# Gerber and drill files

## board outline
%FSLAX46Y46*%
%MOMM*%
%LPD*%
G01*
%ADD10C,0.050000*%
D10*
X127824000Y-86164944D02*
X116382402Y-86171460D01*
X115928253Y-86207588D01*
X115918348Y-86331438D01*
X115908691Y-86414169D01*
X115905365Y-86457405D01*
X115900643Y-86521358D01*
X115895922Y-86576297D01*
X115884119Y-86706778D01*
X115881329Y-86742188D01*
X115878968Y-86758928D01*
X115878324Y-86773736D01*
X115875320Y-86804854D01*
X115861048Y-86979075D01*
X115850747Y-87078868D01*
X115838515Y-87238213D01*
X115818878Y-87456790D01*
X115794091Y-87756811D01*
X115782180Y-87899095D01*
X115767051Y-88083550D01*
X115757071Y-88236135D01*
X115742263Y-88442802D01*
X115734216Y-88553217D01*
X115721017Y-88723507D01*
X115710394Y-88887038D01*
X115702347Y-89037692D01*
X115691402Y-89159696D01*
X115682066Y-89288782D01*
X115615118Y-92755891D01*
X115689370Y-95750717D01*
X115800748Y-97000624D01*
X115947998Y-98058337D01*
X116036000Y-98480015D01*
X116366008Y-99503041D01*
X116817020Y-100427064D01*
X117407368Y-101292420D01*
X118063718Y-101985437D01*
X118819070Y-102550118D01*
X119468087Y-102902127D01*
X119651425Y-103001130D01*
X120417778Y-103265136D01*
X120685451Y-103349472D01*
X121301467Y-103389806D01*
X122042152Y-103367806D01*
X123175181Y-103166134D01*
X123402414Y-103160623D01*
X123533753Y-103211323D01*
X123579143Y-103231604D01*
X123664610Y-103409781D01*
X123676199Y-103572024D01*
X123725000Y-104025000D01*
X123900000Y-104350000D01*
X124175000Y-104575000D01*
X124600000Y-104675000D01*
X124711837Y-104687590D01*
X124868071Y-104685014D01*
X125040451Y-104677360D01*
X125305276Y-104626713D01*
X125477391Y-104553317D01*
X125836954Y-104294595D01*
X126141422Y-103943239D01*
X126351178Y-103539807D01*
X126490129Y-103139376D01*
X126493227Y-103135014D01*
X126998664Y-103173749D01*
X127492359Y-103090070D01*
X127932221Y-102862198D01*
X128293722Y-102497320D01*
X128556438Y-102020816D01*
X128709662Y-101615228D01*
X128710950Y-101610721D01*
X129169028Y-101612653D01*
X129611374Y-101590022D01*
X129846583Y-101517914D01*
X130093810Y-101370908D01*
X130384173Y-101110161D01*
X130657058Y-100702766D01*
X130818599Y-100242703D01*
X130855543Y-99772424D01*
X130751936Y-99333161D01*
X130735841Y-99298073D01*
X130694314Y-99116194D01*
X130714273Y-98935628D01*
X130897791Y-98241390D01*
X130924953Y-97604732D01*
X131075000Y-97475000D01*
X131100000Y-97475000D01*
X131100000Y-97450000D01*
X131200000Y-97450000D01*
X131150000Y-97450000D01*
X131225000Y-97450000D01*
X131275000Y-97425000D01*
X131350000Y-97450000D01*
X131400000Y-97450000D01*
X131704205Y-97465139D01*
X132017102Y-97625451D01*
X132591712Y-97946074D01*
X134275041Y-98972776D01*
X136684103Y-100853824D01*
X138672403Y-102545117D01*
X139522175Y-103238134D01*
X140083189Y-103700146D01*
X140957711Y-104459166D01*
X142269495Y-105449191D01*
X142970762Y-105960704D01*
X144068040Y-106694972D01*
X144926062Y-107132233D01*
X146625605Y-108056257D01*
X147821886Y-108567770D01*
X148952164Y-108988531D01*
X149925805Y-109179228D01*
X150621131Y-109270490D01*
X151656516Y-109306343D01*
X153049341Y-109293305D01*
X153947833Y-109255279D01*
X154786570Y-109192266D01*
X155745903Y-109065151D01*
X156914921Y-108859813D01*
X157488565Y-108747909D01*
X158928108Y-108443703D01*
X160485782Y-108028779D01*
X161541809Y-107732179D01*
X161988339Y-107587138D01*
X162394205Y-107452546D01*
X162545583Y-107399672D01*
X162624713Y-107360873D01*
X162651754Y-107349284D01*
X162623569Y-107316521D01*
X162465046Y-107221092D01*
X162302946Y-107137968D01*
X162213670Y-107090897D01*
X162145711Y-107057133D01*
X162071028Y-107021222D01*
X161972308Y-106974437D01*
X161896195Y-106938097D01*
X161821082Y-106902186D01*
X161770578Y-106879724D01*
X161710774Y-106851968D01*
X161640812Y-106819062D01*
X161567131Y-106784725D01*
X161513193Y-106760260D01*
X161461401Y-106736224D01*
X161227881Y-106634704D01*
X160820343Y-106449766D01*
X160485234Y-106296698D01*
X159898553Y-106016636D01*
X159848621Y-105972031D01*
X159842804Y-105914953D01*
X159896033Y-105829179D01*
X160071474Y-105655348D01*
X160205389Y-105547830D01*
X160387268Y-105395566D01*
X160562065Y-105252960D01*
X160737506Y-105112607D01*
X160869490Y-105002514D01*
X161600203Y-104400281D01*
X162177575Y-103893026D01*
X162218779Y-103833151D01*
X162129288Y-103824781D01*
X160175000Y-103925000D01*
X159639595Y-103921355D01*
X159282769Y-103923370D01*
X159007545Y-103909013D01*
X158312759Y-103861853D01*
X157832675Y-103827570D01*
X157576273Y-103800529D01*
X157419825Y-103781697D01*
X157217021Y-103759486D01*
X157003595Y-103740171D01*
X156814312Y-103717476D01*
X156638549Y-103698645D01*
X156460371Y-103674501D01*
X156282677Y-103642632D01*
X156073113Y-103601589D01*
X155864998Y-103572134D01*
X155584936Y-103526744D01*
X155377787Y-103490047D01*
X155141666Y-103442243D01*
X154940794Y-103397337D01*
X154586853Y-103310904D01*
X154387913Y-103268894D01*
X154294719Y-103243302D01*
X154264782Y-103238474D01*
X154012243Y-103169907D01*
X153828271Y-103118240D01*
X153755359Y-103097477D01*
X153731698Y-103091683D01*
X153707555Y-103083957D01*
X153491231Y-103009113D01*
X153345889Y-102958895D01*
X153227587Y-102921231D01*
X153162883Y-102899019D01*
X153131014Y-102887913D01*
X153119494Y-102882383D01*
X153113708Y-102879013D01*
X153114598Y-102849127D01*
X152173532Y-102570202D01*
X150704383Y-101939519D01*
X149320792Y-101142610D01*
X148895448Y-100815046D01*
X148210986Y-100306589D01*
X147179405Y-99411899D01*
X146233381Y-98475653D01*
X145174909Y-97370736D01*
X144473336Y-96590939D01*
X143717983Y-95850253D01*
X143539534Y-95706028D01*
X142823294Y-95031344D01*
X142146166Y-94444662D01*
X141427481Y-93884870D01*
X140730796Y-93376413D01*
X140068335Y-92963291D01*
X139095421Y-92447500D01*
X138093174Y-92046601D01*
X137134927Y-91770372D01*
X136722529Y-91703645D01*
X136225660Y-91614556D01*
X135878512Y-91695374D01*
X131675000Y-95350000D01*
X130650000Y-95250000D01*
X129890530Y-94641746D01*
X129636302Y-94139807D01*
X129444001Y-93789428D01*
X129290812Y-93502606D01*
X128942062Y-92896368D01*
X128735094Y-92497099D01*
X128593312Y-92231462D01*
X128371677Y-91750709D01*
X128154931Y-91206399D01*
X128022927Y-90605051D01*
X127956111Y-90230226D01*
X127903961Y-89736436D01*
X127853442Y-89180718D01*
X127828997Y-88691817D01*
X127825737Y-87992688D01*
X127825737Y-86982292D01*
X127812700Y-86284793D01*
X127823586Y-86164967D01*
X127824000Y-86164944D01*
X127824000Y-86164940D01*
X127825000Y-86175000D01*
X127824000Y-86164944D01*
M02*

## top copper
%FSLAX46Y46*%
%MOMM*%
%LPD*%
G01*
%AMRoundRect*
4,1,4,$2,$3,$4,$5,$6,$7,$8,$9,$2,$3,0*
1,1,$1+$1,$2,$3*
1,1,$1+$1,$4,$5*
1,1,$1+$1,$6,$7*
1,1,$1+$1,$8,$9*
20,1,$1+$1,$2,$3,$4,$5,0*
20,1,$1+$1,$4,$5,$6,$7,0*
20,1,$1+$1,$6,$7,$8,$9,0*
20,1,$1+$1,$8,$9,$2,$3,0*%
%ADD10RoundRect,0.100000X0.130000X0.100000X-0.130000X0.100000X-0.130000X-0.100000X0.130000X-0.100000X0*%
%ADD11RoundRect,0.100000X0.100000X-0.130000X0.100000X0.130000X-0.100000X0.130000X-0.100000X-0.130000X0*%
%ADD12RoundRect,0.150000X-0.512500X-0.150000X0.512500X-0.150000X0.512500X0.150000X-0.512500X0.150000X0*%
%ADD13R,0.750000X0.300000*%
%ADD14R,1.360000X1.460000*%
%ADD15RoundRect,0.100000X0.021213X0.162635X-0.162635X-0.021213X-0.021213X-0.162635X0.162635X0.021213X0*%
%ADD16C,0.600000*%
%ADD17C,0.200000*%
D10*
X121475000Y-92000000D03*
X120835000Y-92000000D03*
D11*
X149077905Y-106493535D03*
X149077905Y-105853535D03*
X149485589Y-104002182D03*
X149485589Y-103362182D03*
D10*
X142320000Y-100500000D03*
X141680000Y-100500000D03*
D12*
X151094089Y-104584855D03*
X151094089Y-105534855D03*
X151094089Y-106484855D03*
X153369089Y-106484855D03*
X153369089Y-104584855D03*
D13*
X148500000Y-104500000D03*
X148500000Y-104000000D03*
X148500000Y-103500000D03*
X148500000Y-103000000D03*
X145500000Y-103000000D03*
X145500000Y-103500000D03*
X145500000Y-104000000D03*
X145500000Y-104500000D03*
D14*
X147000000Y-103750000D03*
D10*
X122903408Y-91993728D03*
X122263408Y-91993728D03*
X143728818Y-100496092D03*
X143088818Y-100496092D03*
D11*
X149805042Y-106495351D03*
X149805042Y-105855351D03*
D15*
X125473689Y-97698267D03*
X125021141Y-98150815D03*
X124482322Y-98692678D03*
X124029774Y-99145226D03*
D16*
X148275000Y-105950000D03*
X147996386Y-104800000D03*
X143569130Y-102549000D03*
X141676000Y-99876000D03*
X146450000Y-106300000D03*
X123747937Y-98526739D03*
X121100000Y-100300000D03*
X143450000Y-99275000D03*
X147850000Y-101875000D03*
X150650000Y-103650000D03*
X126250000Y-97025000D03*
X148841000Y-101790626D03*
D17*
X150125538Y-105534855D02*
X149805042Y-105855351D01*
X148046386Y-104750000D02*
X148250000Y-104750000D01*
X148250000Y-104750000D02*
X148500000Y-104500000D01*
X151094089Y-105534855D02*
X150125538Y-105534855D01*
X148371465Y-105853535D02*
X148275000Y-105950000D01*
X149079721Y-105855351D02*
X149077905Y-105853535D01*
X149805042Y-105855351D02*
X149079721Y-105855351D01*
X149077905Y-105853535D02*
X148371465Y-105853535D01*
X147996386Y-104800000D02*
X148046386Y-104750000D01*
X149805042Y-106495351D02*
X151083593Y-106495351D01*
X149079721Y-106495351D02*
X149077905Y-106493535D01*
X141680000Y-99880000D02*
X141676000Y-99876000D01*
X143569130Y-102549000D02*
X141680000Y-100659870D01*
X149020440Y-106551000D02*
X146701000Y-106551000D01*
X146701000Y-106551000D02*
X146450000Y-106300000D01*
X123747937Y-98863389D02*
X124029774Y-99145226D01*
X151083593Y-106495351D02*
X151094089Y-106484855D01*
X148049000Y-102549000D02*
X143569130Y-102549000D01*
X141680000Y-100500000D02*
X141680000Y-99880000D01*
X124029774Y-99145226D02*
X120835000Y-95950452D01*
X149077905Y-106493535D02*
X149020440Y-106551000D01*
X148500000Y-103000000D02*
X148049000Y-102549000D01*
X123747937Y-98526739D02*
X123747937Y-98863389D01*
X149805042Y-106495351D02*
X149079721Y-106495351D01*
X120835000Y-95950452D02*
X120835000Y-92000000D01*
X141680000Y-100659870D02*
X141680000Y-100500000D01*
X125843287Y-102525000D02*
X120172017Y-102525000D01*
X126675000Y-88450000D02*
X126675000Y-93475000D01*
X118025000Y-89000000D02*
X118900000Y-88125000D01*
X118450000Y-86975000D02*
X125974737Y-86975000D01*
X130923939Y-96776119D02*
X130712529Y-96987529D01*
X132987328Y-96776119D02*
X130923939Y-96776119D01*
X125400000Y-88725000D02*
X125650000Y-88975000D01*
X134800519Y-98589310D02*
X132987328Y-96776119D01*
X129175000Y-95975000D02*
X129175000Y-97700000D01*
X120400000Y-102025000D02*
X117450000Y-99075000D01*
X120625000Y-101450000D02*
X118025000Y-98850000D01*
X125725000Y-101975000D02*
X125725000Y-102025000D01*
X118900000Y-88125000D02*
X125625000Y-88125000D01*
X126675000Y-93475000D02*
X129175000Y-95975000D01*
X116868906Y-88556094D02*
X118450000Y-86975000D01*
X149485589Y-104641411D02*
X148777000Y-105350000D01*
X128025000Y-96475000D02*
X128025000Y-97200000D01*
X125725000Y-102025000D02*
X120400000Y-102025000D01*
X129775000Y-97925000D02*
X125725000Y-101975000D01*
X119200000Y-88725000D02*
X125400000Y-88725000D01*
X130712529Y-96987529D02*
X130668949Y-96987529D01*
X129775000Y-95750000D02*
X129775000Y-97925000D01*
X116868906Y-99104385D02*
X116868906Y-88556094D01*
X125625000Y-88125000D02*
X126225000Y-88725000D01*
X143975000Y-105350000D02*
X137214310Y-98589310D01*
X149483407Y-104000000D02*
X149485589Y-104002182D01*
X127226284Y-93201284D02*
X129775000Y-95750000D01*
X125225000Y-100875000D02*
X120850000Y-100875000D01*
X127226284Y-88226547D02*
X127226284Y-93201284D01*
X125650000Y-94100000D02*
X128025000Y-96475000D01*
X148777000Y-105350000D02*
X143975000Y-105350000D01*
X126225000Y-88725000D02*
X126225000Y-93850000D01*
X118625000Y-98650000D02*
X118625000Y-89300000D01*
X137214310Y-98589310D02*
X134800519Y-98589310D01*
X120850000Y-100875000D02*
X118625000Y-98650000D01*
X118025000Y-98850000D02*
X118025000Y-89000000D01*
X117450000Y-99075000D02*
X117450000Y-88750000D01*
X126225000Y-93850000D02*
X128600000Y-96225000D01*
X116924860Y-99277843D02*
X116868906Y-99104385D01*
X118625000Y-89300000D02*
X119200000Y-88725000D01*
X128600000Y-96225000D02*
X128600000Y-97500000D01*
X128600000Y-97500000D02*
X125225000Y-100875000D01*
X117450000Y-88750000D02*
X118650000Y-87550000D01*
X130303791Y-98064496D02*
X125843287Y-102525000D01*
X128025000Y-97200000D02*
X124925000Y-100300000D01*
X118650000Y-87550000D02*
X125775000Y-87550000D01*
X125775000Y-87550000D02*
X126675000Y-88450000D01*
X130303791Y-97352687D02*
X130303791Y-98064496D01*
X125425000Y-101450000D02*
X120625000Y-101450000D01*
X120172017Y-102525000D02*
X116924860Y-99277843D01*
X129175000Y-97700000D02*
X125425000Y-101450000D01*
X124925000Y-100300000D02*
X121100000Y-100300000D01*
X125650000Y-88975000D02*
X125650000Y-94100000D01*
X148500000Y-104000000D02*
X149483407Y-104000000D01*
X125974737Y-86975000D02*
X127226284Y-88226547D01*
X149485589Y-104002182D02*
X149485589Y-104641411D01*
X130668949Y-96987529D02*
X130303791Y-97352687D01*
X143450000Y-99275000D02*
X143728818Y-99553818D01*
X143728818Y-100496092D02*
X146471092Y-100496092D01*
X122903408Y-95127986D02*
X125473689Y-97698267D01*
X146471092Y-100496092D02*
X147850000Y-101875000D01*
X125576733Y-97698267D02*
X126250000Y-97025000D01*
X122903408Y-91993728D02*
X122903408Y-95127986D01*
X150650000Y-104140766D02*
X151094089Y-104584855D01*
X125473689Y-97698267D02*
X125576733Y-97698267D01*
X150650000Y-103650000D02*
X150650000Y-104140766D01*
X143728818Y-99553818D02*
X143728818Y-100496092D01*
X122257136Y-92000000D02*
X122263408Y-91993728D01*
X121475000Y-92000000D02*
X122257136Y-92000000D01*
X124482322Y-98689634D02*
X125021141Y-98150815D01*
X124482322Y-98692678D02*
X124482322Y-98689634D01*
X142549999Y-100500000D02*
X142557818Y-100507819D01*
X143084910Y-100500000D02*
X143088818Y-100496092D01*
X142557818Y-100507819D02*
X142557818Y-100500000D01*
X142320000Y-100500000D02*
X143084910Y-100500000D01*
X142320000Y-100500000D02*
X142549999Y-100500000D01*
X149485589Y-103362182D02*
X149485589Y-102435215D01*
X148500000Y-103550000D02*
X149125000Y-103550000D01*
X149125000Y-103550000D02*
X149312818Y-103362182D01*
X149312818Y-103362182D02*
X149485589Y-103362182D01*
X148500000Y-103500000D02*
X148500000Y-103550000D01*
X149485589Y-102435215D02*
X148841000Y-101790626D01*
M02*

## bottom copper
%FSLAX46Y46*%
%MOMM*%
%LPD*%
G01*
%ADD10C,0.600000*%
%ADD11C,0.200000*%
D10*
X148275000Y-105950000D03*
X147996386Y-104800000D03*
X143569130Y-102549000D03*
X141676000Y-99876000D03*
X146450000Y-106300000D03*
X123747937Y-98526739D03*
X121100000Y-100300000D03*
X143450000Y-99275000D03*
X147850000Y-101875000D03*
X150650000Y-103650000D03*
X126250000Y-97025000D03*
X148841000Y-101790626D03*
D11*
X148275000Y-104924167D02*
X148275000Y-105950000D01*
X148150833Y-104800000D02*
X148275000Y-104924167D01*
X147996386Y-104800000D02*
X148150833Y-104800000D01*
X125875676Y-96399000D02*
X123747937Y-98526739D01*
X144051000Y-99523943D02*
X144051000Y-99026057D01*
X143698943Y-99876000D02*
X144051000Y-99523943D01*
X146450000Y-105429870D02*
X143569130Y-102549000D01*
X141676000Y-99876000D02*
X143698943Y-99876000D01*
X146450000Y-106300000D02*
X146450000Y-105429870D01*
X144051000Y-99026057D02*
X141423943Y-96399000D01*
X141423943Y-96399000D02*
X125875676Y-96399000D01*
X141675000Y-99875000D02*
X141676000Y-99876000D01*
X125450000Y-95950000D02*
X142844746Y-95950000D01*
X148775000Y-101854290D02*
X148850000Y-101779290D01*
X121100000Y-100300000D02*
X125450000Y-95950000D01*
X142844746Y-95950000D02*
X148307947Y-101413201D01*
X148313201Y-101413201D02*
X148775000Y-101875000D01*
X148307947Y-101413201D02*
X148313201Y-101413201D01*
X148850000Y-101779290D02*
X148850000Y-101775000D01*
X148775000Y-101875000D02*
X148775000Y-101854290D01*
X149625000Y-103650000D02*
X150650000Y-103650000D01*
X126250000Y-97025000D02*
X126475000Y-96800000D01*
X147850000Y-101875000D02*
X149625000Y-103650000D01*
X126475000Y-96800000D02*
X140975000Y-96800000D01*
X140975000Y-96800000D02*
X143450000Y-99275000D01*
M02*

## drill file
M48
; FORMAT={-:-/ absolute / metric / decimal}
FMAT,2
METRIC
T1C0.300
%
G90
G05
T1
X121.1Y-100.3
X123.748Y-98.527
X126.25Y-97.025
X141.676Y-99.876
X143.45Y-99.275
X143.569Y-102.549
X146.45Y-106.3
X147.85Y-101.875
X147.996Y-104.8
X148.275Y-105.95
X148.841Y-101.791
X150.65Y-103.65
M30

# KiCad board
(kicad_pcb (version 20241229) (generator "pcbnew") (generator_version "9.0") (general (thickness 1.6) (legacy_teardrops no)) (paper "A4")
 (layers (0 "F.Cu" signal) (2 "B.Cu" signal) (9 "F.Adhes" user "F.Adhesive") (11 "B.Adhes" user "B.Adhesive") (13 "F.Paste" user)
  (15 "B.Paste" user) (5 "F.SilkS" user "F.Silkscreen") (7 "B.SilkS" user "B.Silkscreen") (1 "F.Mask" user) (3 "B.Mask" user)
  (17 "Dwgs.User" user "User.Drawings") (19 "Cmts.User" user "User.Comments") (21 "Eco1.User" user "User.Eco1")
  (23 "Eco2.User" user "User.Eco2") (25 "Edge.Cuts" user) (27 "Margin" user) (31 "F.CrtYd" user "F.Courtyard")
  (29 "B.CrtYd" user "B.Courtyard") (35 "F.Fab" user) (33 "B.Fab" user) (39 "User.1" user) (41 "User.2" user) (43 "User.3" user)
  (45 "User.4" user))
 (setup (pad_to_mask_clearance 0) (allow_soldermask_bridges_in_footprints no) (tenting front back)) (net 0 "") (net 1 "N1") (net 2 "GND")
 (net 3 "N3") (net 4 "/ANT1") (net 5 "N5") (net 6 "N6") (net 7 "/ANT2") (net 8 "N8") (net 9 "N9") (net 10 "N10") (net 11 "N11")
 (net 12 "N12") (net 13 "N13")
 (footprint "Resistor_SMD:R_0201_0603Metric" (layer "F.Cu") (at 121.155 92 180)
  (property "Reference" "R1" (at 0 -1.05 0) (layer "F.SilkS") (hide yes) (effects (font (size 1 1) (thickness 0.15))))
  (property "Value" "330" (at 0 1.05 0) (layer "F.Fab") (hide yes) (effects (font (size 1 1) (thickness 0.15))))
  (pad "" smd roundrect (at -0.345 0 180) (size 0.318 0.36) (layers "F.Paste") (roundrect_rratio 0.25))
  (pad "" smd roundrect (at 0.345 0 180) (size 0.318 0.36) (layers "F.Paste") (roundrect_rratio 0.25))
  (pad "1" smd roundrect (at -0.32 0 180) (size 0.46 0.4) (layers "F.Cu" "F.Mask") (roundrect_rratio 0.25) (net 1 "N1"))
  (pad "2" smd roundrect (at 0.32 0 180) (size 0.46 0.4) (layers "F.Cu" "F.Mask") (roundrect_rratio 0.25) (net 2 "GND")))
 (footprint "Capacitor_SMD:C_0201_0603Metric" (layer "F.Cu") (at 149.077905 106.173535 90)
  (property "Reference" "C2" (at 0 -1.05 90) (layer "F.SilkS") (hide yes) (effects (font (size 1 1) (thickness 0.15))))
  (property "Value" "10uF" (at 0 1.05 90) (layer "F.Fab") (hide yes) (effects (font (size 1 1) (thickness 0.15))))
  (pad "" smd roundrect (at -0.345 0 90) (size 0.318 0.36) (layers "F.Paste") (roundrect_rratio 0.25))
  (pad "" smd roundrect (at 0.345 0 90) (size 0.318 0.36) (layers "F.Paste") (roundrect_rratio 0.25))
  (pad "1" smd roundrect (at -0.32 0 90) (size 0.46 0.4) (layers "F.Cu" "F.Mask") (roundrect_rratio 0.25) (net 2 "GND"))
  (pad "2" smd roundrect (at 0.32 0 90) (size 0.46 0.4) (layers "F.Cu" "F.Mask") (roundrect_rratio 0.25) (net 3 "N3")))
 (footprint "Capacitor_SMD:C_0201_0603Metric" (layer "F.Cu") (at 149.485589 103.682182 90)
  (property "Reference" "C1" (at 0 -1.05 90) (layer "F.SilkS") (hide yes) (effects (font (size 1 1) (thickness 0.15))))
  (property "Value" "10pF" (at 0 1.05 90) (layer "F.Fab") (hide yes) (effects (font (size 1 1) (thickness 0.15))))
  (pad "" smd roundrect (at -0.345 0 90) (size 0.318 0.36) (layers "F.Paste") (roundrect_rratio 0.25))
  (pad "" smd roundrect (at 0.345 0 90) (size 0.318 0.36) (layers "F.Paste") (roundrect_rratio 0.25))
  (pad "1" smd roundrect (at -0.32 0 90) (size 0.46 0.4) (layers "F.Cu" "F.Mask") (roundrect_rratio 0.25) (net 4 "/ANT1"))
  (pad "2" smd roundrect (at 0.32 0 90) (size 0.46 0.4) (layers "F.Cu" "F.Mask") (roundrect_rratio 0.25) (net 4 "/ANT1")))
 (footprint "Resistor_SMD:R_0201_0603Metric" (layer "F.Cu") (at 142 100.5 180)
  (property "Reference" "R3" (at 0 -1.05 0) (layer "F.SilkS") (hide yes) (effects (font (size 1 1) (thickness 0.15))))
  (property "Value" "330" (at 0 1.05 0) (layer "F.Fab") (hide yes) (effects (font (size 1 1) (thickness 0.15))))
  (pad "" smd roundrect (at -0.345 0 180) (size 0.318 0.36) (layers "F.Paste") (roundrect_rratio 0.25))
  (pad "" smd roundrect (at 0.345 0 180) (size 0.318 0.36) (layers "F.Paste") (roundrect_rratio 0.25))
  (pad "1" smd roundrect (at -0.32 0 180) (size 0.46 0.4) (layers "F.Cu" "F.Mask") (roundrect_rratio 0.25) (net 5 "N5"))
  (pad "2" smd roundrect (at 0.32 0 180) (size 0.46 0.4) (layers "F.Cu" "F.Mask") (roundrect_rratio 0.25) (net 2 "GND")))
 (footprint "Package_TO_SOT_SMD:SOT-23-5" (layer "F.Cu") (at 152.231589 105.534855)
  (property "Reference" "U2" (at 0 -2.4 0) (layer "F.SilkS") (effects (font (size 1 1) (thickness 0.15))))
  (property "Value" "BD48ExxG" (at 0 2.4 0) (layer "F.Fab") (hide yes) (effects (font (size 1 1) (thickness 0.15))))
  (pad "1" smd roundrect (at -1.1375 -0.95) (size 1.325 0.6) (layers "F.Cu" "F.Mask" "F.Paste") (roundrect_rratio 0.25) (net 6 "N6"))
  (pad "2" smd roundrect (at -1.1375 0) (size 1.325 0.6) (layers "F.Cu" "F.Mask" "F.Paste") (roundrect_rratio 0.25) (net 3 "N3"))
  (pad "3" smd roundrect (at -1.1375 0.95) (size 1.325 0.6) (layers "F.Cu" "F.Mask" "F.Paste") (roundrect_rratio 0.25) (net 2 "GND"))
  (pad "4" smd roundrect (at 1.1375 0.95) (size 1.325 0.6) (layers "F.Cu" "F.Mask" "F.Paste") (roundrect_rratio 0.25))
  (pad "5" smd roundrect (at 1.1375 -0.95) (size 1.325 0.6) (layers "F.Cu" "F.Mask" "F.Paste") (roundrect_rratio 0.25)))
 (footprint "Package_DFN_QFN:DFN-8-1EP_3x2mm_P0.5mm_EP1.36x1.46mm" (layer "F.Cu") (at 147 103.75 180)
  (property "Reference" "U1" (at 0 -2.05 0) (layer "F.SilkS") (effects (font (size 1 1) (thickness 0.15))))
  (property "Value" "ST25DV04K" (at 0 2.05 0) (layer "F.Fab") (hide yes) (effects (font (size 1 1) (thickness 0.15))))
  (pad "" smd rect (at -0.325 -0.375 180) (size 0.5 0.6) (layers "F.Paste"))
  (pad "" smd rect (at -0.325 0.375 180) (size 0.5 0.6) (layers "F.Paste"))
  (pad "" smd rect (at 0.325 -0.375 180) (size 0.5 0.6) (layers "F.Paste"))
  (pad "" smd rect (at 0.325 0.375 180) (size 0.5 0.6) (layers "F.Paste"))
  (pad "1" smd rect (at -1.5 -0.75 180) (size 0.75 0.3) (layers "F.Cu" "F.Mask" "F.Paste") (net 3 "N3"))
  (pad "2" smd rect (at -1.5 -0.25 180) (size 0.75 0.3) (layers "F.Cu" "F.Mask" "F.Paste") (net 4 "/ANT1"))
  (pad "3" smd rect (at -1.5 0.25 180) (size 0.75 0.3) (layers "F.Cu" "F.Mask" "F.Paste") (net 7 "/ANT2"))
  (pad "4" smd rect (at -1.5 0.75 180) (size 0.75 0.3) (layers "F.Cu" "F.Mask" "F.Paste") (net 2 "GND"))
  (pad "5" smd rect (at 1.5 0.75 180) (size 0.75 0.3) (layers "F.Cu" "F.Mask" "F.Paste") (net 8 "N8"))
  (pad "6" smd rect (at 1.5 0.25 180) (size 0.75 0.3) (layers "F.Cu" "F.Mask" "F.Paste") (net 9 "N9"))
  (pad "7" smd rect (at 1.5 -0.25 180) (size 0.75 0.3) (layers "F.Cu" "F.Mask" "F.Paste") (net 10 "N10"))
  (pad "8" smd rect (at 1.5 -0.75 180) (size 0.75 0.3) (layers "F.Cu" "F.Mask" "F.Paste") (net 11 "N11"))
  (pad "9" smd rect (at 0 0 180) (size 1.36 1.46) (layers "F.Cu" "F.Mask") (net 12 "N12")))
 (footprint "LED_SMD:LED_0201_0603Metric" (layer "F.Cu") (at 122.583408 91.993728 180)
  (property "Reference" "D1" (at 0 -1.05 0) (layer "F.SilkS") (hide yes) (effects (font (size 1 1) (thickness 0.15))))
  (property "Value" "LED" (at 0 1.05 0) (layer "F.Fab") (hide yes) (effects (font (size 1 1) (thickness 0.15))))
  (pad "" smd roundrect (at -0.345 0 180) (size 0.318 0.36) (layers "F.Paste") (roundrect_rratio 0.25))
  (pad "" smd roundrect (at 0.345 0 180) (size 0.318 0.36) (layers "F.Paste") (roundrect_rratio 0.25))
  (pad "1" smd roundrect (at -0.32 0 180) (size 0.46 0.4) (layers "F.Cu" "F.Mask") (roundrect_rratio 0.25) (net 6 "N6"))
  (pad "2" smd roundrect (at 0.32 0 180) (size 0.46 0.4) (layers "F.Cu" "F.Mask") (roundrect_rratio 0.25) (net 1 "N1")))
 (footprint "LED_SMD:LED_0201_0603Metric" (layer "F.Cu") (at 143.408818 100.496092 180)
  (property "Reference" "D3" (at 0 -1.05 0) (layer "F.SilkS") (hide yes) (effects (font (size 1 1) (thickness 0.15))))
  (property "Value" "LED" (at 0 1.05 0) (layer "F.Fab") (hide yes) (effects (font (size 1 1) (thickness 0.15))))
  (pad "" smd roundrect (at -0.345 0 180) (size 0.318 0.36) (layers "F.Paste") (roundrect_rratio 0.25))
  (pad "" smd roundrect (at 0.345 0 180) (size 0.318 0.36) (layers "F.Paste") (roundrect_rratio 0.25))
  (pad "1" smd roundrect (at -0.32 0 180) (size 0.46 0.4) (layers "F.Cu" "F.Mask") (roundrect_rratio 0.25) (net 6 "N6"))
  (pad "2" smd roundrect (at 0.32 0 180) (size 0.46 0.4) (layers "F.Cu" "F.Mask") (roundrect_rratio 0.25) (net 5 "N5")))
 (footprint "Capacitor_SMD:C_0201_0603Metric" (layer "F.Cu") (at 149.805042 106.175351 90)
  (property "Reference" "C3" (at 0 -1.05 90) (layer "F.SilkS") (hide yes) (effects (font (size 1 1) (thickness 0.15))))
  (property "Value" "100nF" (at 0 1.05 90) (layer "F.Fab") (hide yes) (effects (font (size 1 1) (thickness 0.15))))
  (pad "" smd roundrect (at -0.345 0 90) (size 0.318 0.36) (layers "F.Paste") (roundrect_rratio 0.25))
  (pad "" smd roundrect (at 0.345 0 90) (size 0.318 0.36) (layers "F.Paste") (roundrect_rratio 0.25))
  (pad "1" smd roundrect (at -0.32 0 90) (size 0.46 0.4) (layers "F.Cu" "F.Mask") (roundrect_rratio 0.25) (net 2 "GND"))
  (pad "2" smd roundrect (at 0.32 0 90) (size 0.46 0.4) (layers "F.Cu" "F.Mask") (roundrect_rratio 0.25) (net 3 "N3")))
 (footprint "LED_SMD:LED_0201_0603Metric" (layer "F.Cu") (at 125.247415 97.924541 -135)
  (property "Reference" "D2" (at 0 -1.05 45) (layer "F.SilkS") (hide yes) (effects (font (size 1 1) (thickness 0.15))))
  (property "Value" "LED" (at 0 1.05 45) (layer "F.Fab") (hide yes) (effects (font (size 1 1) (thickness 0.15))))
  (pad "" smd roundrect (at -0.345 0 225) (size 0.318 0.36) (layers "F.Paste") (roundrect_rratio 0.25))
  (pad "" smd roundrect (at 0.345 0 225) (size 0.318 0.36) (layers "F.Paste") (roundrect_rratio 0.25))
  (pad "1" smd roundrect (at -0.32 0 225) (size 0.46 0.4) (layers "F.Cu" "F.Mask") (roundrect_rratio 0.25) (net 6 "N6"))
  (pad "2" smd roundrect (at 0.32 0 225) (size 0.46 0.4) (layers "F.Cu" "F.Mask") (roundrect_rratio 0.25) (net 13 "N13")))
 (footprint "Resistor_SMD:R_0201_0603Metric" (layer "F.Cu") (at 124.256048 98.918952 -135)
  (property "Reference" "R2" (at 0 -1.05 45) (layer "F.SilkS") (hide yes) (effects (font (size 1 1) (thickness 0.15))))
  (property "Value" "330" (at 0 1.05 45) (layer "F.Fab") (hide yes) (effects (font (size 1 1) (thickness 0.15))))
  (pad "" smd roundrect (at -0.345 0 225) (size 0.318 0.36) (layers "F.Paste") (roundrect_rratio 0.25))
  (pad "" smd roundrect (at 0.345 0 225) (size 0.318 0.36) (layers "F.Paste") (roundrect_rratio 0.25))
  (pad "1" smd roundrect (at -0.32 0 225) (size 0.46 0.4) (layers "F.Cu" "F.Mask") (roundrect_rratio 0.25) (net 13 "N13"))
  (pad "2" smd roundrect (at 0.32 0 225) (size 0.46 0.4) (layers "F.Cu" "F.Mask") (roundrect_rratio 0.25) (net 2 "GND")))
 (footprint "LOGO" (layer "F.Cu") (at 139 99.5)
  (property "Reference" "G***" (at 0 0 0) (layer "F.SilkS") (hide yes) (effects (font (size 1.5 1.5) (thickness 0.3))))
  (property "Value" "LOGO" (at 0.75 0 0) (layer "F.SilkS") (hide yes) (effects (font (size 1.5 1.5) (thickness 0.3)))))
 (gr_poly
  (pts (xy 127.824 86.164944) (xy 116.382402 86.17146) (xy 115.928253 86.207588) (xy 115.918348 86.331438) (xy 115.908691 86.414169)
   (xy 115.905365 86.457405) (xy 115.900643 86.521358) (xy 115.895922 86.576297) (xy 115.884119 86.706778) (xy 115.881329 86.742188)
   (xy 115.878968 86.758928) (xy 115.878324 86.773736) (xy 115.87532 86.804854) (xy 115.861048 86.979075) (xy 115.850747 87.078868)
   (xy 115.838515 87.238213) (xy 115.818878 87.45679) (xy 115.794091 87.756811) (xy 115.78218 87.899095) (xy 115.767051 88.08355)
   (xy 115.757071 88.236135) (xy 115.742263 88.442802) (xy 115.734216 88.553217) (xy 115.721017 88.723507) (xy 115.710394 88.887038)
   (xy 115.702347 89.037692) (xy 115.691402 89.159696) (xy 115.682066 89.288782) (xy 115.615118 92.755891) (xy 115.68937 95.750717)
   (xy 115.800748 97.000624) (xy 115.947998 98.058337) (xy 116.036 98.480015) (xy 116.366008 99.503041) (xy 116.81702 100.427064)
   (xy 117.407368 101.29242) (xy 118.063718 101.985437) (xy 118.81907 102.550118) (xy 119.468087 102.902127) (xy 119.651425 103.00113)
   (xy 120.417778 103.265136) (xy 120.685451 103.349472) (xy 121.301467 103.389806) (xy 122.042152 103.367806) (xy 123.175181 103.166134)
   (xy 123.402414 103.160623) (xy 123.533753 103.211323) (xy 123.579143 103.231604) (xy 123.66461 103.409781) (xy 123.676199 103.572024)
   (xy 123.725 104.025) (xy 123.9 104.35) (xy 124.175 104.575) (xy 124.6 104.675) (xy 124.711837 104.68759) (xy 124.868071 104.685014)
   (xy 125.040451 104.67736) (xy 125.305276 104.626713) (xy 125.477391 104.553317) (xy 125.836954 104.294595) (xy 126.141422 103.943239)
   (xy 126.351178 103.539807) (xy 126.490129 103.139376) (xy 126.493227 103.135014) (xy 126.998664 103.173749) (xy 127.492359 103.09007)
   (xy 127.932221 102.862198) (xy 128.293722 102.49732) (xy 128.556438 102.020816) (xy 128.709662 101.615228) (xy 128.71095 101.610721)
   (xy 129.169028 101.612653) (xy 129.611374 101.590022) (xy 129.846583 101.517914) (xy 130.09381 101.370908) (xy 130.384173 101.110161)
   (xy 130.657058 100.702766) (xy 130.818599 100.242703) (xy 130.855543 99.772424) (xy 130.751936 99.333161) (xy 130.735841 99.298073)
   (xy 130.694314 99.116194) (xy 130.714273 98.935628) (xy 130.897791 98.24139) (xy 130.924953 97.604732) (xy 131.075 97.475)
   (xy 131.1 97.475) (xy 131.1 97.45) (xy 131.2 97.45) (xy 131.15 97.45) (xy 131.225 97.45) (xy 131.275 97.425) (xy 131.35 97.45)
   (xy 131.4 97.45) (xy 131.704205 97.465139) (xy 132.017102 97.625451) (xy 132.591712 97.946074) (xy 134.275041 98.972776)
   (xy 136.684103 100.853824) (xy 138.672403 102.545117) (xy 139.522175 103.238134) (xy 140.083189 103.700146) (xy 140.957711 104.459166)
   (xy 142.269495 105.449191) (xy 142.970762 105.960704) (xy 144.06804 106.694972) (xy 144.926062 107.132233) (xy 146.625605 108.056257)
   (xy 147.821886 108.56777) (xy 148.952164 108.988531) (xy 149.925805 109.179228) (xy 150.621131 109.27049) (xy 151.656516 109.306343)
   (xy 153.049341 109.293305) (xy 153.947833 109.255279) (xy 154.78657 109.192266) (xy 155.745903 109.065151) (xy 156.914921 108.859813)
   (xy 157.488565 108.747909) (xy 158.928108 108.443703) (xy 160.485782 108.028779) (xy 161.541809 107.732179) (xy 161.988339 107.587138)
   (xy 162.394205 107.452546) (xy 162.545583 107.399672) (xy 162.624713 107.360873) (xy 162.651754 107.349284) (xy 162.623569 107.316521)
   (xy 162.465046 107.221092) (xy 162.302946 107.137968) (xy 162.21367 107.090897) (xy 162.145711 107.057133) (xy 162.071028 107.021222)
   (xy 161.972308 106.974437) (xy 161.896195 106.938097) (xy 161.821082 106.902186) (xy 161.770578 106.879724) (xy 161.710774 106.851968)
   (xy 161.640812 106.819062) (xy 161.567131 106.784725) (xy 161.513193 106.76026) (xy 161.461401 106.736224) (xy 161.227881 106.634704)
   (xy 160.820343 106.449766) (xy 160.485234 106.296698) (xy 159.898553 106.016636) (xy 159.848621 105.972031) (xy 159.842804 105.914953)
   (xy 159.896033 105.829179) (xy 160.071474 105.655348) (xy 160.205389 105.54783) (xy 160.387268 105.395566) (xy 160.562065 105.25296)
   (xy 160.737506 105.112607) (xy 160.86949 105.002514) (xy 161.600203 104.400281) (xy 162.177575 103.893026) (xy 162.218779 103.833151)
   (xy 162.129288 103.824781) (xy 160.175 103.925) (xy 159.639595 103.921355) (xy 159.282769 103.92337) (xy 159.007545 103.909013)
   (xy 158.312759 103.861853) (xy 157.832675 103.82757) (xy 157.576273 103.800529) (xy 157.419825 103.781697) (xy 157.217021 103.759486)
   (xy 157.003595 103.740171) (xy 156.814312 103.717476) (xy 156.638549 103.698645) (xy 156.460371 103.674501) (xy 156.282677 103.642632)
   (xy 156.073113 103.601589) (xy 155.864998 103.572134) (xy 155.584936 103.526744) (xy 155.377787 103.490047) (xy 155.141666 103.442243)
   (xy 154.940794 103.397337) (xy 154.586853 103.310904) (xy 154.387913 103.268894) (xy 154.294719 103.243302) (xy 154.264782 103.238474)
   (xy 154.012243 103.169907) (xy 153.828271 103.11824) (xy 153.755359 103.097477) (xy 153.731698 103.091683) (xy 153.707555 103.083957)
   (xy 153.491231 103.009113) (xy 153.345889 102.958895) (xy 153.227587 102.921231) (xy 153.162883 102.899019) (xy 153.131014 102.887913)
   (xy 153.119494 102.882383) (xy 153.113708 102.879013) (xy 153.114598 102.849127) (xy 152.173532 102.570202) (xy 150.704383 101.939519)
   (xy 149.320792 101.14261) (xy 148.895448 100.815046) (xy 148.210986 100.306589) (xy 147.179405 99.411899) (xy 146.233381 98.475653)
   (xy 145.174909 97.370736) (xy 144.473336 96.590939) (xy 143.717983 95.850253) (xy 143.539534 95.706028) (xy 142.823294 95.031344)
   (xy 142.146166 94.444662) (xy 141.427481 93.88487) (xy 140.730796 93.376413) (xy 140.068335 92.963291) (xy 139.095421 92.4475)
   (xy 138.093174 92.046601) (xy 137.134927 91.770372) (xy 136.722529 91.703645) (xy 136.22566 91.614556) (xy 135.878512 91.695374)
   (xy 131.675 95.35) (xy 130.65 95.25) (xy 129.89053 94.641746) (xy 129.636302 94.139807) (xy 129.444001 93.789428)
   (xy 129.290812 93.502606) (xy 128.942062 92.896368) (xy 128.735094 92.497099) (xy 128.593312 92.231462) (xy 128.371677 91.750709)
   (xy 128.154931 91.206399) (xy 128.022927 90.605051) (xy 127.956111 90.230226) (xy 127.903961 89.736436) (xy 127.853442 89.180718)
   (xy 127.828997 88.691817) (xy 127.825737 87.992688) (xy 127.825737 86.982292) (xy 127.8127 86.284793) (xy 127.823586 86.164967)
   (xy 127.824 86.164944) (xy 127.824 86.16494) (xy 127.825 86.175))
  (stroke (width 0.05) (type solid)) (fill no) (layer "Edge.Cuts"))
 (segment (start 150.125538 105.534855) (end 149.805042 105.855351) (width 0.2) (layer "F.Cu") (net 3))
 (segment (start 148.046386 104.75) (end 148.25 104.75) (width 0.2) (layer "F.Cu") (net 3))
 (segment (start 148.25 104.75) (end 148.5 104.5) (width 0.2) (layer "F.Cu") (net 3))
 (segment (start 151.094089 105.534855) (end 150.125538 105.534855) (width 0.2) (layer "F.Cu") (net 3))
 (segment (start 148.371465 105.853535) (end 148.275 105.95) (width 0.2) (layer "F.Cu") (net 3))
 (segment (start 149.079721 105.855351) (end 149.077905 105.853535) (width 0.2) (layer "F.Cu") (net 3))
 (segment (start 149.805042 105.855351) (end 149.079721 105.855351) (width 0.2) (layer "F.Cu") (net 3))
 (segment (start 149.077905 105.853535) (end 148.371465 105.853535) (width 0.2) (layer "F.Cu") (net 3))
 (segment (start 147.996386 104.8) (end 148.046386 104.75) (width 0.2) (layer "F.Cu") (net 3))
 (via (at 148.275 105.95) (size 0.6) (drill 0.3) (layers "F.Cu" "B.Cu") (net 3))
 (via (at 147.996386 104.8) (size 0.6) (drill 0.3) (layers "F.Cu" "B.Cu") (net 3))
 (segment (start 148.275 104.924167) (end 148.275 105.95) (width 0.2) (layer "B.Cu") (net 3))
 (segment (start 148.150833 104.8) (end 148.275 104.924167) (width 0.2) (layer "B.Cu") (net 3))
 (segment (start 147.996386 104.8) (end 148.150833 104.8) (width 0.2) (layer "B.Cu") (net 3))
 (segment (start 149.805042 106.495351) (end 151.083593 106.495351) (width 0.2) (layer "F.Cu") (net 2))
 (segment (start 149.079721 106.495351) (end 149.077905 106.493535) (width 0.2) (layer "F.Cu") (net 2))
 (segment (start 141.68 99.88) (end 141.676 99.876) (width 0.2) (layer "F.Cu") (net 2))
 (segment (start 143.56913 102.549) (end 141.68 100.65987) (width 0.2) (layer "F.Cu") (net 2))
 (segment (start 149.02044 106.551) (end 146.701 106.551) (width 0.2) (layer "F.Cu") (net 2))
 (segment (start 146.701 106.551) (end 146.45 106.3) (width 0.2) (layer "F.Cu") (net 2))
 (segment (start 123.747937 98.863389) (end 124.029774 99.145226) (width 0.2) (layer "F.Cu") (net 2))
 (segment (start 151.083593 106.495351) (end 151.094089 106.484855) (width 0.2) (layer "F.Cu") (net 2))
 (segment (start 148.049 102.549) (end 143.56913 102.549) (width 0.2) (layer "F.Cu") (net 2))
 (segment (start 141.68 100.5) (end 141.68 99.88) (width 0.2) (layer "F.Cu") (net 2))
 (segment (start 124.029774 99.145226) (end 120.835 95.950452) (width 0.2) (layer "F.Cu") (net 2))
 (segment (start 149.077905 106.493535) (end 149.02044 106.551) (width 0.2) (layer "F.Cu") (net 2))
 (segment (start 148.5 103) (end 148.049 102.549) (width 0.2) (layer "F.Cu") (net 2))
 (segment (start 123.747937 98.526739) (end 123.747937 98.863389) (width 0.2) (layer "F.Cu") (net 2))
 (segment (start 149.805042 106.495351) (end 149.079721 106.495351) (width 0.2) (layer "F.Cu") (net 2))
 (segment (start 120.835 95.950452) (end 120.835 92) (width 0.2) (layer "F.Cu") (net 2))
 (segment (start 141.68 100.65987) (end 141.68 100.5) (width 0.2) (layer "F.Cu") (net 2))
 (via (at 143.56913 102.549) (size 0.6) (drill 0.3) (layers "F.Cu" "B.Cu") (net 2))
 (via (at 141.676 99.876) (size 0.6) (drill 0.3) (layers "F.Cu" "B.Cu") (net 2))
 (via (at 146.45 106.3) (size 0.6) (drill 0.3) (layers "F.Cu" "B.Cu") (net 2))
 (via (at 123.747937 98.526739) (size 0.6) (drill 0.3) (layers "F.Cu" "B.Cu") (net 2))
 (segment (start 125.875676 96.399) (end 123.747937 98.526739) (width 0.2) (layer "B.Cu") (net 2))
 (segment (start 144.051 99.523943) (end 144.051 99.026057) (width 0.2) (layer "B.Cu") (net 2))
 (segment (start 143.698943 99.876) (end 144.051 99.523943) (width 0.2) (layer "B.Cu") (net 2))
 (segment (start 146.45 105.42987) (end 143.56913 102.549) (width 0.2) (layer "B.Cu") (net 2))
 (segment (start 141.676 99.876) (end 143.698943 99.876) (width 0.2) (layer "B.Cu") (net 2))
 (segment (start 146.45 106.3) (end 146.45 105.42987) (width 0.2) (layer "B.Cu") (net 2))
 (segment (start 144.051 99.026057) (end 141.423943 96.399) (width 0.2) (layer "B.Cu") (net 2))
 (segment (start 141.423943 96.399) (end 125.875676 96.399) (width 0.2) (layer "B.Cu") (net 2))
 (segment (start 141.675 99.875) (end 141.676 99.876) (width 0.2) (layer "B.Cu") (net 2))
 (segment (start 125.843287 102.525) (end 120.172017 102.525) (width 0.2) (layer "F.Cu") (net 4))
 (segment (start 126.675 88.45) (end 126.675 93.475) (width 0.2) (layer "F.Cu") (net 4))
 (segment (start 118.025 89) (end 118.9 88.125) (width 0.2) (layer "F.Cu") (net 4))
 (segment (start 118.45 86.975) (end 125.974737 86.975) (width 0.2) (layer "F.Cu") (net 4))
 (segment (start 130.923939 96.776119) (end 130.712529 96.987529) (width 0.2) (layer "F.Cu") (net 4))
 (segment (start 132.987328 96.776119) (end 130.923939 96.776119) (width 0.2) (layer "F.Cu") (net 4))
 (segment (start 125.4 88.725) (end 125.65 88.975) (width 0.2) (layer "F.Cu") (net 4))
 (segment (start 134.800519 98.58931) (end 132.987328 96.776119) (width 0.2) (layer "F.Cu") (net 4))
 (segment (start 129.175 95.975) (end 129.175 97.7) (width 0.2) (layer "F.Cu") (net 4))
 (segment (start 120.4 102.025) (end 117.45 99.075) (width 0.2) (layer "F.Cu") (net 4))
 (segment (start 120.625 101.45) (end 118.025 98.85) (width 0.2) (layer "F.Cu") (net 4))
 (segment (start 125.725 101.975) (end 125.725 102.025) (width 0.2) (layer "F.Cu") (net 4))
 (segment (start 118.9 88.125) (end 125.625 88.125) (width 0.2) (layer "F.Cu") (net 4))
 (segment (start 126.675 93.475) (end 129.175 95.975) (width 0.2) (layer "F.Cu") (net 4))
 (segment (start 116.868906 88.556094) (end 118.45 86.975) (width 0.2) (layer "F.Cu") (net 4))
 (segment (start 149.485589 104.641411) (end 148.777 105.35) (width 0.2) (layer "F.Cu") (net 4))
 (segment (start 128.025 96.475) (end 128.025 97.2) (width 0.2) (layer "F.Cu") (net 4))
 (segment (start 125.725 102.025) (end 120.4 102.025) (width 0.2) (layer "F.Cu") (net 4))
 (segment (start 129.775 97.925) (end 125.725 101.975) (width 0.2) (layer "F.Cu") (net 4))
 (segment (start 119.2 88.725) (end 125.4 88.725) (width 0.2) (layer "F.Cu") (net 4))
 (segment (start 130.712529 96.987529) (end 130.668949 96.987529) (width 0.2) (layer "F.Cu") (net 4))
 (segment (start 129.775 95.75) (end 129.775 97.925) (width 0.2) (layer "F.Cu") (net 4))
 (segment (start 116.868906 99.104385) (end 116.868906 88.556094) (width 0.2) (layer "F.Cu") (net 4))
 (segment (start 125.625 88.125) (end 126.225 88.725) (width 0.2) (layer "F.Cu") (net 4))
 (segment (start 143.975 105.35) (end 137.21431 98.58931) (width 0.2) (layer "F.Cu") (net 4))
 (segment (start 149.483407 104) (end 149.485589 104.002182) (width 0.2) (layer "F.Cu") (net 4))
 (segment (start 127.226284 93.201284) (end 129.775 95.75) (width 0.2) (layer "F.Cu") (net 4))
 (segment (start 125.225 100.875) (end 120.85 100.875) (width 0.2) (layer "F.Cu") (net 4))
 (segment (start 127.226284 88.226547) (end 127.226284 93.201284) (width 0.2) (layer "F.Cu") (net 4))
 (segment (start 125.65 94.1) (end 128.025 96.475) (width 0.2) (layer "F.Cu") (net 4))
 (segment (start 148.777 105.35) (end 143.975 105.35) (width 0.2) (layer "F.Cu") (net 4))
 (segment (start 126.225 88.725) (end 126.225 93.85) (width 0.2) (layer "F.Cu") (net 4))
 (segment (start 118.625 98.65) (end 118.625 89.3) (width 0.2) (layer "F.Cu") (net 4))
 (segment (start 137.21431 98.58931) (end 134.800519 98.58931) (width 0.2) (layer "F.Cu") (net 4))
 (segment (start 120.85 100.875) (end 118.625 98.65) (width 0.2) (layer "F.Cu") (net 4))
 (segment (start 118.025 98.85) (end 118.025 89) (width 0.2) (layer "F.Cu") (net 4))
 (segment (start 117.45 99.075) (end 117.45 88.75) (width 0.2) (layer "F.Cu") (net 4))
 (segment (start 126.225 93.85) (end 128.6 96.225) (width 0.2) (layer "F.Cu") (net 4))
 (segment (start 116.92486 99.277843) (end 116.868906 99.104385) (width 0.2) (layer "F.Cu") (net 4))
 (segment (start 118.625 89.3) (end 119.2 88.725) (width 0.2) (layer "F.Cu") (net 4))
 (segment (start 128.6 96.225) (end 128.6 97.5) (width 0.2) (layer "F.Cu") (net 4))
 (segment (start 128.6 97.5) (end 125.225 100.875) (width 0.2) (layer "F.Cu") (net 4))
 (segment (start 117.45 88.75) (end 118.65 87.55) (width 0.2) (layer "F.Cu") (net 4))
 (segment (start 130.303791 98.064496) (end 125.843287 102.525) (width 0.2) (layer "F.Cu") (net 4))
 (segment (start 128.025 97.2) (end 124.925 100.3) (width 0.2) (layer "F.Cu") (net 4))
 (segment (start 118.65 87.55) (end 125.775 87.55) (width 0.2) (layer "F.Cu") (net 4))
 (segment (start 125.775 87.55) (end 126.675 88.45) (width 0.2) (layer "F.Cu") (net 4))
 (segment (start 130.303791 97.352687) (end 130.303791 98.064496) (width 0.2) (layer "F.Cu") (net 4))
 (segment (start 125.425 101.45) (end 120.625 101.45) (width 0.2) (layer "F.Cu") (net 4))
 (segment (start 120.172017 102.525) (end 116.92486 99.277843) (width 0.2) (layer "F.Cu") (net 4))
 (segment (start 129.175 97.7) (end 125.425 101.45) (width 0.2) (layer "F.Cu") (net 4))
 (segment (start 124.925 100.3) (end 121.1 100.3) (width 0.2) (layer "F.Cu") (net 4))
 (segment (start 125.65 88.975) (end 125.65 94.1) (width 0.2) (layer "F.Cu") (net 4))
 (segment (start 148.5 104) (end 149.483407 104) (width 0.2) (layer "F.Cu") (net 4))
 (segment (start 125.974737 86.975) (end 127.226284 88.226547) (width 0.2) (layer "F.Cu") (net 4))
 (segment (start 149.485589 104.002182) (end 149.485589 104.641411) (width 0.2) (layer "F.Cu") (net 4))
 (segment (start 130.668949 96.987529) (end 130.303791 97.352687) (width 0.2) (layer "F.Cu") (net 4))
 (via (at 121.1 100.3) (size 0.6) (drill 0.3) (layers "F.Cu" "B.Cu") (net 4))
 (segment (start 125.45 95.95) (end 142.844746 95.95) (width 0.2) (layer "B.Cu") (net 4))
 (segment (start 148.775 101.85429) (end 148.85 101.77929) (width 0.2) (layer "B.Cu") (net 4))
 (segment (start 121.1 100.3) (end 125.45 95.95) (width 0.2) (layer "B.Cu") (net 4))
 (segment (start 142.844746 95.95) (end 148.307947 101.413201) (width 0.2) (layer "B.Cu") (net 4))
 (segment (start 148.313201 101.413201) (end 148.775 101.875) (width 0.2) (layer "B.Cu") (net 4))
 (segment (start 148.307947 101.413201) (end 148.313201 101.413201) (width 0.2) (layer "B.Cu") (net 4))
 (segment (start 148.85 101.77929) (end 148.85 101.775) (width 0.2) (layer "B.Cu") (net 4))
 (segment (start 148.775 101.875) (end 148.775 101.85429) (width 0.2) (layer "B.Cu") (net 4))
 (segment (start 143.45 99.275) (end 143.728818 99.553818) (width 0.2) (layer "F.Cu") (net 6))
 (segment (start 143.728818 100.496092) (end 146.471092 100.496092) (width 0.2) (layer "F.Cu") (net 6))
 (segment (start 122.903408 95.127986) (end 125.473689 97.698267) (width 0.2) (layer "F.Cu") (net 6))
 (segment (start 146.471092 100.496092) (end 147.85 101.875) (width 0.2) (layer "F.Cu") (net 6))
 (segment (start 125.576733 97.698267) (end 126.25 97.025) (width 0.2) (layer "F.Cu") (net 6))
 (segment (start 122.903408 91.993728) (end 122.903408 95.127986) (width 0.2) (layer "F.Cu") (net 6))
 (segment (start 150.65 104.140766) (end 151.094089 104.584855) (width 0.2) (layer "F.Cu") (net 6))
 (segment (start 125.473689 97.698267) (end 125.576733 97.698267) (width 0.2) (layer "F.Cu") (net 6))
 (segment (start 150.65 103.65) (end 150.65 104.140766) (width 0.2) (layer "F.Cu") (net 6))
 (segment (start 143.728818 99.553818) (end 143.728818 100.496092) (width 0.2) (layer "F.Cu") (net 6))
 (via (at 143.45 99.275) (size 0.6) (drill 0.3) (layers "F.Cu" "B.Cu") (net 6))
 (via (at 147.85 101.875) (size 0.6) (drill 0.3) (layers "F.Cu" "B.Cu") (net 6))
 (via (at 150.65 103.65) (size 0.6) (drill 0.3) (layers "F.Cu" "B.Cu") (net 6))
 (via (at 126.25 97.025) (size 0.6) (drill 0.3) (layers "F.Cu" "B.Cu") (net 6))
 (segment (start 149.625 103.65) (end 150.65 103.65) (width 0.2) (layer "B.Cu") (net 6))
 (segment (start 126.25 97.025) (end 126.475 96.8) (width 0.2) (layer "B.Cu") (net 6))
 (segment (start 147.85 101.875) (end 149.625 103.65) (width 0.2) (layer "B.Cu") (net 6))
 (segment (start 126.475 96.8) (end 140.975 96.8) (width 0.2) (layer "B.Cu") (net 6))
 (segment (start 140.975 96.8) (end 143.45 99.275) (width 0.2) (layer "B.Cu") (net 6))
 (segment (start 122.257136 92) (end 122.263408 91.993728) (width 0.2) (layer "F.Cu") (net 1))
 (segment (start 121.475 92) (end 122.257136 92) (width 0.2) (layer "F.Cu") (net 1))
 (segment (start 124.482322 98.689634) (end 125.021141 98.150815) (width 0.2) (layer "F.Cu") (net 13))
 (segment (start 124.482322 98.692678) (end 124.482322 98.689634) (width 0.2) (layer "F.Cu") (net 13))
 (segment (start 142.549999 100.5) (end 142.557818 100.507819) (width 0.2) (layer "F.Cu") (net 5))
 (segment (start 143.08491 100.5) (end 143.088818 100.496092) (width 0.2) (layer "F.Cu") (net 5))
 (segment (start 142.557818 100.507819) (end 142.557818 100.5) (width 0.2) (layer "F.Cu") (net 5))
 (segment (start 142.32 100.5) (end 143.08491 100.5) (width 0.2) (layer "F.Cu") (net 5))
 (segment (start 142.32 100.5) (end 142.549999 100.5) (width 0.2) (layer "F.Cu") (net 5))
 (segment (start 149.485589 103.362182) (end 149.485589 102.435215) (width 0.2) (layer "F.Cu") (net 7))
 (segment (start 148.5 103.55) (end 149.125 103.55) (width 0.2) (layer "F.Cu") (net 7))
 (segment (start 149.125 103.55) (end 149.312818 103.362182) (width 0.2) (layer "F.Cu") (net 7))
 (segment (start 149.312818 103.362182) (end 149.485589 103.362182) (width 0.2) (layer "F.Cu") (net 7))
 (segment (start 148.5 103.5) (end 148.5 103.55) (width 0.2) (layer "F.Cu") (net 7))
 (segment (start 149.485589 102.435215) (end 148.841 101.790626) (width 0.2) (layer "F.Cu") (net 7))
 (via (at 148.841 101.790626) (size 0.6) (drill 0.3) (layers "F.Cu" "B.Cu") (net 7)))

